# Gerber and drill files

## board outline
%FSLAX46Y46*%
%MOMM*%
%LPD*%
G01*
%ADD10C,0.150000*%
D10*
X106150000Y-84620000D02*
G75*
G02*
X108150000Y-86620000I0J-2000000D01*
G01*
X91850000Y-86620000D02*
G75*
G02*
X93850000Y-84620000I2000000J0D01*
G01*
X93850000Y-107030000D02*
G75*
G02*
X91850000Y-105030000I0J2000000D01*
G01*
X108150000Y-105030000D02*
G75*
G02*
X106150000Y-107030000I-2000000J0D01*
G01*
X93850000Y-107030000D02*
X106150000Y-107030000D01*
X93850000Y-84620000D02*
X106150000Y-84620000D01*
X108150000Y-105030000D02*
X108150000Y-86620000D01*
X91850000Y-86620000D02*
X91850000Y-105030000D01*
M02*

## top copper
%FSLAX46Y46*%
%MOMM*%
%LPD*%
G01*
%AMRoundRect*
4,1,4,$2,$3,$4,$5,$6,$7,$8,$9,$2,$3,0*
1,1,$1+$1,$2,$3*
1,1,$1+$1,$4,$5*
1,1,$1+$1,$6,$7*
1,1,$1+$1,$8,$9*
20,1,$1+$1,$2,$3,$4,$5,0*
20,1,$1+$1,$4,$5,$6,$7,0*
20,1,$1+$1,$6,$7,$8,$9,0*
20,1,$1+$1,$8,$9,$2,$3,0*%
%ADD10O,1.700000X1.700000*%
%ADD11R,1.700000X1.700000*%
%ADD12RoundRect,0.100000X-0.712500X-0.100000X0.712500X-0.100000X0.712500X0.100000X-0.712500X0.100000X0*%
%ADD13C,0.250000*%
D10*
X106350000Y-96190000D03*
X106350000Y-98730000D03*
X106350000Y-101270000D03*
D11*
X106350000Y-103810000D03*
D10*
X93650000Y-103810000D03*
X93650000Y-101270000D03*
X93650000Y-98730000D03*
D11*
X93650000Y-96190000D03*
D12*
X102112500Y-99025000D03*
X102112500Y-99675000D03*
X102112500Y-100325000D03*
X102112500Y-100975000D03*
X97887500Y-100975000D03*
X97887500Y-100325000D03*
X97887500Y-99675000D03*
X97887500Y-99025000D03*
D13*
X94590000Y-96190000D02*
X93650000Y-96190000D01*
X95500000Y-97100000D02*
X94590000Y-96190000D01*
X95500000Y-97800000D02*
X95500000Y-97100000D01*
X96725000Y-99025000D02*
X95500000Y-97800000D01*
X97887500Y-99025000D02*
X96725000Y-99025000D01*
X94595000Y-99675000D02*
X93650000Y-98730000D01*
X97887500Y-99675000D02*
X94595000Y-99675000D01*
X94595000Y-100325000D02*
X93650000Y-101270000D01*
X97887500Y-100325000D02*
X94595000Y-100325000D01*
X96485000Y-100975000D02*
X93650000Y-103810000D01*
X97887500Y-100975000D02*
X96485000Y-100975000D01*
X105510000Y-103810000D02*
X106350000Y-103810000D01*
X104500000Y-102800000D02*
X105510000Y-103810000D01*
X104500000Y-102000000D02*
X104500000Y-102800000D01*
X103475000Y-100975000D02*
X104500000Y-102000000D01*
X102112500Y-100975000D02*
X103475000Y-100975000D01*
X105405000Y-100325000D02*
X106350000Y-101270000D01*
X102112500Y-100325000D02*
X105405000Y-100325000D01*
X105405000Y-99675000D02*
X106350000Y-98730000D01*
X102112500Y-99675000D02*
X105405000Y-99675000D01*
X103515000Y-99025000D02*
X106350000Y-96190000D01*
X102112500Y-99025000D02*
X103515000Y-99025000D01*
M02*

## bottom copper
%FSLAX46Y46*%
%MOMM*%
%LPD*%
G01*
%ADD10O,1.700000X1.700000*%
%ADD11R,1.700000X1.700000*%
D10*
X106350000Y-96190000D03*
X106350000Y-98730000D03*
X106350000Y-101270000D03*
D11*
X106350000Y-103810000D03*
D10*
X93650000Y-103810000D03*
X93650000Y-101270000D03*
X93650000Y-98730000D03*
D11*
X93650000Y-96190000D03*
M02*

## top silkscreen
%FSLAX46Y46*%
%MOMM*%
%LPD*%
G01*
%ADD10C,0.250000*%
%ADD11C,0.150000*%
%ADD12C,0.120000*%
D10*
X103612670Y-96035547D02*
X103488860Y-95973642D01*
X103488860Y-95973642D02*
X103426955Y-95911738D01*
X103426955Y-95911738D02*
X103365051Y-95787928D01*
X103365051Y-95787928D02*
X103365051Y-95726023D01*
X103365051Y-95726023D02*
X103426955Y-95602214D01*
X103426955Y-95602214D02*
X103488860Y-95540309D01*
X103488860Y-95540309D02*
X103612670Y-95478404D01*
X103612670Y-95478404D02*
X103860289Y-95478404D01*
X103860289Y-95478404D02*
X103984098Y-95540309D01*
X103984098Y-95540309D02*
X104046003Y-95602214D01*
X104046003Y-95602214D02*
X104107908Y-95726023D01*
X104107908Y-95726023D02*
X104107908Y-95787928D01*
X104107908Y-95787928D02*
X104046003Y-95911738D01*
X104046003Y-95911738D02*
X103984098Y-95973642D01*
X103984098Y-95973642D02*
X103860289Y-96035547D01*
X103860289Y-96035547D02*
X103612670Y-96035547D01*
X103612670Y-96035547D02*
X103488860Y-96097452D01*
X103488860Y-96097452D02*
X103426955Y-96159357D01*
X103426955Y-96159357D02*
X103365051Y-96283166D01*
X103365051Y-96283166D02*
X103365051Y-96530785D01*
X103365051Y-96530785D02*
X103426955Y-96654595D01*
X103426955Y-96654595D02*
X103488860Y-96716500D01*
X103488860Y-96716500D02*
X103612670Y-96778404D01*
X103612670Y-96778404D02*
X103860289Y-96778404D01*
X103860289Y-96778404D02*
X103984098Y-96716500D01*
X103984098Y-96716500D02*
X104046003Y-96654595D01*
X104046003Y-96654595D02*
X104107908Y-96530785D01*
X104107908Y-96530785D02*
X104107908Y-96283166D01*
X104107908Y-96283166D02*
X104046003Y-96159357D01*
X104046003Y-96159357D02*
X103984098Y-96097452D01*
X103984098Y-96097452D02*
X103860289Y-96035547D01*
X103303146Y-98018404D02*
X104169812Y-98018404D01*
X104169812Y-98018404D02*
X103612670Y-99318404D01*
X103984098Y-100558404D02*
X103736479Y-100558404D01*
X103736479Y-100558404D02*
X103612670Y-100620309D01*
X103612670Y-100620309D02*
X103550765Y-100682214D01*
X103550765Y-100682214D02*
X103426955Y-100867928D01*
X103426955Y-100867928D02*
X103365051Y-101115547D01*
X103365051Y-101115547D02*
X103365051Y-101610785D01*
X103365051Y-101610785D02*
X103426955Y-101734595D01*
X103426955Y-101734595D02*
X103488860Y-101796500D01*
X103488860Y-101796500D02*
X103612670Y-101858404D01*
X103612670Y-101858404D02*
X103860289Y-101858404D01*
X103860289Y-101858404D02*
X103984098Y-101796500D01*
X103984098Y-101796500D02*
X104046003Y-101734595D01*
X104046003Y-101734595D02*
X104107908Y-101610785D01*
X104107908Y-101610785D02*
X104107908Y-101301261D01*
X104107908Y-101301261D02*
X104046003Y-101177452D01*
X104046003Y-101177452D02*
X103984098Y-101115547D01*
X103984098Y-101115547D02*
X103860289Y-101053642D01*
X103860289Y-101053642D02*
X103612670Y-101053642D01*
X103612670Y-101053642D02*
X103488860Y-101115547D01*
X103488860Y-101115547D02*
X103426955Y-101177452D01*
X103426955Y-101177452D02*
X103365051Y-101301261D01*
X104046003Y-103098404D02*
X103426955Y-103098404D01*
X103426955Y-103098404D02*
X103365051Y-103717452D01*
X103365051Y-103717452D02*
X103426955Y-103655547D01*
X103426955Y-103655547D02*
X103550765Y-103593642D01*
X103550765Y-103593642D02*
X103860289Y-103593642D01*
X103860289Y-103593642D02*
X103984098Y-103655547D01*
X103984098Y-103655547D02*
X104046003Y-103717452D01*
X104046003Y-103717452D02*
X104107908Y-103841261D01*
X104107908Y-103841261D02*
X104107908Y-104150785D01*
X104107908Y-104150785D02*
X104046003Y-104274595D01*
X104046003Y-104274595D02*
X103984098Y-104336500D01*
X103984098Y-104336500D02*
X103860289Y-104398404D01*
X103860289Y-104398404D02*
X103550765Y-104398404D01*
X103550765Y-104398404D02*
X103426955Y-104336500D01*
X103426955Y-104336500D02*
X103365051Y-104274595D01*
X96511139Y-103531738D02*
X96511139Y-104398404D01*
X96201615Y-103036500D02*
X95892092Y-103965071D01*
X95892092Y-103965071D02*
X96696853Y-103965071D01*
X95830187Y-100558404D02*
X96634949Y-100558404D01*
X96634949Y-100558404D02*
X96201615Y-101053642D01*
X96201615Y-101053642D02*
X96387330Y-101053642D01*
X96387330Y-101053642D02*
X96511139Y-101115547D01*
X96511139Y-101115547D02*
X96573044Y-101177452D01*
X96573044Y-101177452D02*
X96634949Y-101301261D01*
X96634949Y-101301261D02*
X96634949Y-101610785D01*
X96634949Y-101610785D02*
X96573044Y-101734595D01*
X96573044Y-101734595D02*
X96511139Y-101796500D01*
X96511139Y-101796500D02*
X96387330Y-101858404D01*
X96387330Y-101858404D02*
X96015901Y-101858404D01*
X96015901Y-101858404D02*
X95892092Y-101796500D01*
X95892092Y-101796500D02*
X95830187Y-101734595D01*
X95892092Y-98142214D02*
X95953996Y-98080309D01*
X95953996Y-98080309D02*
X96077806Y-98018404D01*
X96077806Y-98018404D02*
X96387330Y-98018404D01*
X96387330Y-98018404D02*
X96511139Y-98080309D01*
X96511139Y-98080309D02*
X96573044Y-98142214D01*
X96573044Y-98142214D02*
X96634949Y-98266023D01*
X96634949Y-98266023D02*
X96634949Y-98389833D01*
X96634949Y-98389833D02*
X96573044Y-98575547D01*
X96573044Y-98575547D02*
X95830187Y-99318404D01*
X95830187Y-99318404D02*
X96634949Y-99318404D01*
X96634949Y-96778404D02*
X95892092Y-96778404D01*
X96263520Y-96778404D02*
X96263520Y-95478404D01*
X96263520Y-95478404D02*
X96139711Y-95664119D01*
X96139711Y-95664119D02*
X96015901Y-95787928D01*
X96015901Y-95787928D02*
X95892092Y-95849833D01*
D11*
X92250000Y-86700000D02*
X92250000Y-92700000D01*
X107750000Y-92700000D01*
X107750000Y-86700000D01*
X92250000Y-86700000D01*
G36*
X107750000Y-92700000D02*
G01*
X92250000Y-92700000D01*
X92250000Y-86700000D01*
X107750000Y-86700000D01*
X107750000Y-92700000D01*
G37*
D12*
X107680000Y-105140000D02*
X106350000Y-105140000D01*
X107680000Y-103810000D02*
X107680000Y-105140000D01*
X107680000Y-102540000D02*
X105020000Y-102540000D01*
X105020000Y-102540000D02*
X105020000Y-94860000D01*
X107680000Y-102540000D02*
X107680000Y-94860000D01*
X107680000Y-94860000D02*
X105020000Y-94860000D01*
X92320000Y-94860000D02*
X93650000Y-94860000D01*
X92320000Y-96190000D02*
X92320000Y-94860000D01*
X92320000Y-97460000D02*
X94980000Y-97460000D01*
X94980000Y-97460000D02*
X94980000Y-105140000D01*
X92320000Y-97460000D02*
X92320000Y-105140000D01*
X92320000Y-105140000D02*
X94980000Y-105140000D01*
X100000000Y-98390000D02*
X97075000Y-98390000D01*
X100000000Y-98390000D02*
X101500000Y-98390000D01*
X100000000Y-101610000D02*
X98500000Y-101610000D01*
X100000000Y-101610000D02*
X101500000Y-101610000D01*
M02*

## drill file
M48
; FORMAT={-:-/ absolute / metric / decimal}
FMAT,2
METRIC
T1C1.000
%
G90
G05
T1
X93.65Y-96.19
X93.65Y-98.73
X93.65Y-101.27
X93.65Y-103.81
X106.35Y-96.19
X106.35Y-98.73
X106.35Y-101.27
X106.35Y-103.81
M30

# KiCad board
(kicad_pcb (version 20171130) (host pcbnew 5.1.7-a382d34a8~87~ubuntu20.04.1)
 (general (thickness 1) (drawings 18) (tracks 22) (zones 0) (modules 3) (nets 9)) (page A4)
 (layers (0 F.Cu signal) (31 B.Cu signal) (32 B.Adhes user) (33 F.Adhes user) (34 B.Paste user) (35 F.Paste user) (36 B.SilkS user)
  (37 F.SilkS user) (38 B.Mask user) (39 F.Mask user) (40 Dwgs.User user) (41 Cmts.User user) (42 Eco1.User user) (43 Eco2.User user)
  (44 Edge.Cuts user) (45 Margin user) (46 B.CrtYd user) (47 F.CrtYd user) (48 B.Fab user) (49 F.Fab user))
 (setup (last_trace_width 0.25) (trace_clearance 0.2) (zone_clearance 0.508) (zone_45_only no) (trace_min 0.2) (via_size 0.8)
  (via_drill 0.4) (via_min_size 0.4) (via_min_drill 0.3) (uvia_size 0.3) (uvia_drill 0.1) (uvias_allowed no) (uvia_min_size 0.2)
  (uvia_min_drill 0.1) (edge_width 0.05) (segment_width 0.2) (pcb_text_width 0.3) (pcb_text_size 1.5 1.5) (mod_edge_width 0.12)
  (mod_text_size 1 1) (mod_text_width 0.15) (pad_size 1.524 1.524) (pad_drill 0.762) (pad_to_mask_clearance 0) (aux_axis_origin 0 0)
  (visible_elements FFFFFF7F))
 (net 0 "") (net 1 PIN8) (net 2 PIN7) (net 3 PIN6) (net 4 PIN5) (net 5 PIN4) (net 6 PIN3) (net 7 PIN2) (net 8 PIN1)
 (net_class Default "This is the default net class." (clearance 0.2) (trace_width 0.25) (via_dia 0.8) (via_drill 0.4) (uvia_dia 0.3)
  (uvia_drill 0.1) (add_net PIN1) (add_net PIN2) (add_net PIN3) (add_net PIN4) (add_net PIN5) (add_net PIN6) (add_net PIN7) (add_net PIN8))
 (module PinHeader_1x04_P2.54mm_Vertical (layer F.Cu) (at 106.35 103.81 180)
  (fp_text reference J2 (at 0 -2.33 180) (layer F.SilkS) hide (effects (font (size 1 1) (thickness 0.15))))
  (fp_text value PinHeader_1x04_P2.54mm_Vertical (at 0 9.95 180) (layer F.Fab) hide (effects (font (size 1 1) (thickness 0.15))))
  (fp_line (start -1.33 -1.33) (end 0 -1.33) (layer F.SilkS) (width 0.12))
  (fp_line (start -1.33 0) (end -1.33 -1.33) (layer F.SilkS) (width 0.12))
  (fp_line (start -1.33 1.27) (end 1.33 1.27) (layer F.SilkS) (width 0.12))
  (fp_line (start 1.33 1.27) (end 1.33 8.95) (layer F.SilkS) (width 0.12))
  (fp_line (start -1.33 1.27) (end -1.33 8.95) (layer F.SilkS) (width 0.12))
  (fp_line (start -1.33 8.95) (end 1.33 8.95) (layer F.SilkS) (width 0.12))
  (pad 4 thru_hole oval (at 0 7.62 180) (size 1.7 1.7) (drill 1) (layers *.Cu *.Mask) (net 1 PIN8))
  (pad 3 thru_hole oval (at 0 5.08 180) (size 1.7 1.7) (drill 1) (layers *.Cu *.Mask) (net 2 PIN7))
  (pad 2 thru_hole oval (at 0 2.54 180) (size 1.7 1.7) (drill 1) (layers *.Cu *.Mask) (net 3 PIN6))
  (pad 1 thru_hole rect (at 0 0 180) (size 1.7 1.7) (drill 1) (layers *.Cu *.Mask) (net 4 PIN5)))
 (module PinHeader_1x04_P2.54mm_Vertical (layer F.Cu) (at 93.65 96.19)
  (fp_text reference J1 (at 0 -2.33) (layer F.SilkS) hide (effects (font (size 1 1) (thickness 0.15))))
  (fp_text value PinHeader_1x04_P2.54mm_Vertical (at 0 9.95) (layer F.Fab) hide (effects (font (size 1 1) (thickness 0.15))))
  (fp_line (start -1.33 -1.33) (end 0 -1.33) (layer F.SilkS) (width 0.12))
  (fp_line (start -1.33 0) (end -1.33 -1.33) (layer F.SilkS) (width 0.12))
  (fp_line (start -1.33 1.27) (end 1.33 1.27) (layer F.SilkS) (width 0.12))
  (fp_line (start 1.33 1.27) (end 1.33 8.95) (layer F.SilkS) (width 0.12))
  (fp_line (start -1.33 1.27) (end -1.33 8.95) (layer F.SilkS) (width 0.12))
  (fp_line (start -1.33 8.95) (end 1.33 8.95) (layer F.SilkS) (width 0.12))
  (pad 4 thru_hole oval (at 0 7.62) (size 1.7 1.7) (drill 1) (layers *.Cu *.Mask) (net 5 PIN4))
  (pad 3 thru_hole oval (at 0 5.08) (size 1.7 1.7) (drill 1) (layers *.Cu *.Mask) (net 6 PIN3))
  (pad 2 thru_hole oval (at 0 2.54) (size 1.7 1.7) (drill 1) (layers *.Cu *.Mask) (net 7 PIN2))
  (pad 1 thru_hole rect (at 0 0) (size 1.7 1.7) (drill 1) (layers *.Cu *.Mask) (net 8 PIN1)))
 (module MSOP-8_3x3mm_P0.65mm (layer F.Cu) (at 100 100)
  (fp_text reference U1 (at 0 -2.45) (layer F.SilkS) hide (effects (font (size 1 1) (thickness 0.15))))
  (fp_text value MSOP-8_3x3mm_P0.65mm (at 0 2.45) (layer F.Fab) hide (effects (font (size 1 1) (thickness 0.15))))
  (fp_line (start 0 -1.61) (end -2.925 -1.61) (layer F.SilkS) (width 0.12))
  (fp_line (start 0 -1.61) (end 1.5 -1.61) (layer F.SilkS) (width 0.12))
  (fp_line (start 0 1.61) (end -1.5 1.61) (layer F.SilkS) (width 0.12))
  (fp_line (start 0 1.61) (end 1.5 1.61) (layer F.SilkS) (width 0.12))
  (pad 8 smd roundrect (at 2.1125 -0.975) (size 1.625 0.4) (layers F.Cu F.Paste F.Mask) (roundrect_rratio 0.25) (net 1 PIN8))
  (pad 7 smd roundrect (at 2.1125 -0.325) (size 1.625 0.4) (layers F.Cu F.Paste F.Mask) (roundrect_rratio 0.25) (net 2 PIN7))
  (pad 6 smd roundrect (at 2.1125 0.325) (size 1.625 0.4) (layers F.Cu F.Paste F.Mask) (roundrect_rratio 0.25) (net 3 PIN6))
  (pad 5 smd roundrect (at 2.1125 0.975) (size 1.625 0.4) (layers F.Cu F.Paste F.Mask) (roundrect_rratio 0.25) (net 4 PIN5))
  (pad 4 smd roundrect (at -2.1125 0.975) (size 1.625 0.4) (layers F.Cu F.Paste F.Mask) (roundrect_rratio 0.25) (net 5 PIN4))
  (pad 3 smd roundrect (at -2.1125 0.325) (size 1.625 0.4) (layers F.Cu F.Paste F.Mask) (roundrect_rratio 0.25) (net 6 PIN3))
  (pad 2 smd roundrect (at -2.1125 -0.325) (size 1.625 0.4) (layers F.Cu F.Paste F.Mask) (roundrect_rratio 0.25) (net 7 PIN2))
  (pad 1 smd roundrect (at -2.1125 -0.975) (size 1.625 0.4) (layers F.Cu F.Paste F.Mask) (roundrect_rratio 0.25) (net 8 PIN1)))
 (gr_arc (start 106.15 86.62) (end 106.15 84.62) (angle 90) (layer Edge.Cuts) (width 0.15))
 (gr_arc (start 93.85 86.62) (end 91.85 86.62) (angle 90) (layer Edge.Cuts) (width 0.15))
 (gr_arc (start 93.85 105.03) (end 93.85 107.03) (angle 90) (layer Edge.Cuts) (width 0.15))
 (gr_arc (start 106.15 105.03) (end 108.15 105.03) (angle 90) (layer Edge.Cuts) (width 0.15))
 (gr_line (start 93.85 107.03) (end 106.15 107.03) (layer Edge.Cuts) (width 0.15))
 (gr_line (start 93.85 84.62) (end 106.15 84.62) (layer Edge.Cuts) (width 0.15))
 (gr_line (start 108.15 105.03) (end 108.15 86.62) (layer Edge.Cuts) (width 0.15))
 (gr_line (start 91.85 86.62) (end 91.85 105.03) (layer Edge.Cuts) (width 0.15))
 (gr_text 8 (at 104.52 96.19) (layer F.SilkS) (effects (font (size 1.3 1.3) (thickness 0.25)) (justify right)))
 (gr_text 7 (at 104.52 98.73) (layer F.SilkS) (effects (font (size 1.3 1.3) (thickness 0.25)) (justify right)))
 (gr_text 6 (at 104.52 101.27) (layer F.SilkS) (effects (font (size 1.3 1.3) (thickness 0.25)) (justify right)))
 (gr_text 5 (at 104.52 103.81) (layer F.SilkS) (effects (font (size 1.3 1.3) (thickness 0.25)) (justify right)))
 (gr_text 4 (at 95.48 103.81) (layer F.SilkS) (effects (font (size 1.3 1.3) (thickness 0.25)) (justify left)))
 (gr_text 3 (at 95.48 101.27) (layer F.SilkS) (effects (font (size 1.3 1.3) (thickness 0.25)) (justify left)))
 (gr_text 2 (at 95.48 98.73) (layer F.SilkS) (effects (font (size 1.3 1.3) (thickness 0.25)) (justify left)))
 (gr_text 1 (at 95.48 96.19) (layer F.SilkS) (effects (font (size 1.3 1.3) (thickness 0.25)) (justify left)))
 (gr_poly (pts (xy 92.25 86.7) (xy 92.25 92.7) (xy 107.75 92.7) (xy 107.75 86.7)) (layer F.SilkS) (width 0.15))
 (segment (start 94.59 96.19) (end 93.65 96.19) (width 0.25) (layer F.Cu) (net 8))
 (segment (start 95.5 97.1) (end 94.59 96.19) (width 0.25) (layer F.Cu) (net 8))
 (segment (start 95.5 97.8) (end 95.5 97.1) (width 0.25) (layer F.Cu) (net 8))
 (segment (start 96.725 99.025) (end 95.5 97.8) (width 0.25) (layer F.Cu) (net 8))
 (segment (start 97.8875 99.025) (end 96.725 99.025) (width 0.25) (layer F.Cu) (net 8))
 (segment (start 94.595 99.675) (end 93.65 98.73) (width 0.25) (layer F.Cu) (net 7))
 (segment (start 97.8875 99.675) (end 94.595 99.675) (width 0.25) (layer F.Cu) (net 7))
 (segment (start 94.595 100.325) (end 93.65 101.27) (width 0.25) (layer F.Cu) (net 6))
 (segment (start 97.8875 100.325) (end 94.595 100.325) (width 0.25) (layer F.Cu) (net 6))
 (segment (start 96.485 100.975) (end 93.65 103.81) (width 0.25) (layer F.Cu) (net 5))
 (segment (start 97.8875 100.975) (end 96.485 100.975) (width 0.25) (layer F.Cu) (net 5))
 (segment (start 105.51 103.81) (end 106.35 103.81) (width 0.25) (layer F.Cu) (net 4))
 (segment (start 104.5 102.8) (end 105.51 103.81) (width 0.25) (layer F.Cu) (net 4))
 (segment (start 104.5 102) (end 104.5 102.8) (width 0.25) (layer F.Cu) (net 4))
 (segment (start 103.475 100.975) (end 104.5 102) (width 0.25) (layer F.Cu) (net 4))
 (segment (start 102.1125 100.975) (end 103.475 100.975) (width 0.25) (layer F.Cu) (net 4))
 (segment (start 105.405 100.325) (end 106.35 101.27) (width 0.25) (layer F.Cu) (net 3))
 (segment (start 102.1125 100.325) (end 105.405 100.325) (width 0.25) (layer F.Cu) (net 3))
 (segment (start 105.405 99.675) (end 106.35 98.73) (width 0.25) (layer F.Cu) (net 2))
 (segment (start 102.1125 99.675) (end 105.405 99.675) (width 0.25) (layer F.Cu) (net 2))
 (segment (start 103.515 99.025) (end 106.35 96.19) (width 0.25) (layer F.Cu) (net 1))
 (segment (start 102.1125 99.025) (end 103.515 99.025) (width 0.25) (layer F.Cu) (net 1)))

